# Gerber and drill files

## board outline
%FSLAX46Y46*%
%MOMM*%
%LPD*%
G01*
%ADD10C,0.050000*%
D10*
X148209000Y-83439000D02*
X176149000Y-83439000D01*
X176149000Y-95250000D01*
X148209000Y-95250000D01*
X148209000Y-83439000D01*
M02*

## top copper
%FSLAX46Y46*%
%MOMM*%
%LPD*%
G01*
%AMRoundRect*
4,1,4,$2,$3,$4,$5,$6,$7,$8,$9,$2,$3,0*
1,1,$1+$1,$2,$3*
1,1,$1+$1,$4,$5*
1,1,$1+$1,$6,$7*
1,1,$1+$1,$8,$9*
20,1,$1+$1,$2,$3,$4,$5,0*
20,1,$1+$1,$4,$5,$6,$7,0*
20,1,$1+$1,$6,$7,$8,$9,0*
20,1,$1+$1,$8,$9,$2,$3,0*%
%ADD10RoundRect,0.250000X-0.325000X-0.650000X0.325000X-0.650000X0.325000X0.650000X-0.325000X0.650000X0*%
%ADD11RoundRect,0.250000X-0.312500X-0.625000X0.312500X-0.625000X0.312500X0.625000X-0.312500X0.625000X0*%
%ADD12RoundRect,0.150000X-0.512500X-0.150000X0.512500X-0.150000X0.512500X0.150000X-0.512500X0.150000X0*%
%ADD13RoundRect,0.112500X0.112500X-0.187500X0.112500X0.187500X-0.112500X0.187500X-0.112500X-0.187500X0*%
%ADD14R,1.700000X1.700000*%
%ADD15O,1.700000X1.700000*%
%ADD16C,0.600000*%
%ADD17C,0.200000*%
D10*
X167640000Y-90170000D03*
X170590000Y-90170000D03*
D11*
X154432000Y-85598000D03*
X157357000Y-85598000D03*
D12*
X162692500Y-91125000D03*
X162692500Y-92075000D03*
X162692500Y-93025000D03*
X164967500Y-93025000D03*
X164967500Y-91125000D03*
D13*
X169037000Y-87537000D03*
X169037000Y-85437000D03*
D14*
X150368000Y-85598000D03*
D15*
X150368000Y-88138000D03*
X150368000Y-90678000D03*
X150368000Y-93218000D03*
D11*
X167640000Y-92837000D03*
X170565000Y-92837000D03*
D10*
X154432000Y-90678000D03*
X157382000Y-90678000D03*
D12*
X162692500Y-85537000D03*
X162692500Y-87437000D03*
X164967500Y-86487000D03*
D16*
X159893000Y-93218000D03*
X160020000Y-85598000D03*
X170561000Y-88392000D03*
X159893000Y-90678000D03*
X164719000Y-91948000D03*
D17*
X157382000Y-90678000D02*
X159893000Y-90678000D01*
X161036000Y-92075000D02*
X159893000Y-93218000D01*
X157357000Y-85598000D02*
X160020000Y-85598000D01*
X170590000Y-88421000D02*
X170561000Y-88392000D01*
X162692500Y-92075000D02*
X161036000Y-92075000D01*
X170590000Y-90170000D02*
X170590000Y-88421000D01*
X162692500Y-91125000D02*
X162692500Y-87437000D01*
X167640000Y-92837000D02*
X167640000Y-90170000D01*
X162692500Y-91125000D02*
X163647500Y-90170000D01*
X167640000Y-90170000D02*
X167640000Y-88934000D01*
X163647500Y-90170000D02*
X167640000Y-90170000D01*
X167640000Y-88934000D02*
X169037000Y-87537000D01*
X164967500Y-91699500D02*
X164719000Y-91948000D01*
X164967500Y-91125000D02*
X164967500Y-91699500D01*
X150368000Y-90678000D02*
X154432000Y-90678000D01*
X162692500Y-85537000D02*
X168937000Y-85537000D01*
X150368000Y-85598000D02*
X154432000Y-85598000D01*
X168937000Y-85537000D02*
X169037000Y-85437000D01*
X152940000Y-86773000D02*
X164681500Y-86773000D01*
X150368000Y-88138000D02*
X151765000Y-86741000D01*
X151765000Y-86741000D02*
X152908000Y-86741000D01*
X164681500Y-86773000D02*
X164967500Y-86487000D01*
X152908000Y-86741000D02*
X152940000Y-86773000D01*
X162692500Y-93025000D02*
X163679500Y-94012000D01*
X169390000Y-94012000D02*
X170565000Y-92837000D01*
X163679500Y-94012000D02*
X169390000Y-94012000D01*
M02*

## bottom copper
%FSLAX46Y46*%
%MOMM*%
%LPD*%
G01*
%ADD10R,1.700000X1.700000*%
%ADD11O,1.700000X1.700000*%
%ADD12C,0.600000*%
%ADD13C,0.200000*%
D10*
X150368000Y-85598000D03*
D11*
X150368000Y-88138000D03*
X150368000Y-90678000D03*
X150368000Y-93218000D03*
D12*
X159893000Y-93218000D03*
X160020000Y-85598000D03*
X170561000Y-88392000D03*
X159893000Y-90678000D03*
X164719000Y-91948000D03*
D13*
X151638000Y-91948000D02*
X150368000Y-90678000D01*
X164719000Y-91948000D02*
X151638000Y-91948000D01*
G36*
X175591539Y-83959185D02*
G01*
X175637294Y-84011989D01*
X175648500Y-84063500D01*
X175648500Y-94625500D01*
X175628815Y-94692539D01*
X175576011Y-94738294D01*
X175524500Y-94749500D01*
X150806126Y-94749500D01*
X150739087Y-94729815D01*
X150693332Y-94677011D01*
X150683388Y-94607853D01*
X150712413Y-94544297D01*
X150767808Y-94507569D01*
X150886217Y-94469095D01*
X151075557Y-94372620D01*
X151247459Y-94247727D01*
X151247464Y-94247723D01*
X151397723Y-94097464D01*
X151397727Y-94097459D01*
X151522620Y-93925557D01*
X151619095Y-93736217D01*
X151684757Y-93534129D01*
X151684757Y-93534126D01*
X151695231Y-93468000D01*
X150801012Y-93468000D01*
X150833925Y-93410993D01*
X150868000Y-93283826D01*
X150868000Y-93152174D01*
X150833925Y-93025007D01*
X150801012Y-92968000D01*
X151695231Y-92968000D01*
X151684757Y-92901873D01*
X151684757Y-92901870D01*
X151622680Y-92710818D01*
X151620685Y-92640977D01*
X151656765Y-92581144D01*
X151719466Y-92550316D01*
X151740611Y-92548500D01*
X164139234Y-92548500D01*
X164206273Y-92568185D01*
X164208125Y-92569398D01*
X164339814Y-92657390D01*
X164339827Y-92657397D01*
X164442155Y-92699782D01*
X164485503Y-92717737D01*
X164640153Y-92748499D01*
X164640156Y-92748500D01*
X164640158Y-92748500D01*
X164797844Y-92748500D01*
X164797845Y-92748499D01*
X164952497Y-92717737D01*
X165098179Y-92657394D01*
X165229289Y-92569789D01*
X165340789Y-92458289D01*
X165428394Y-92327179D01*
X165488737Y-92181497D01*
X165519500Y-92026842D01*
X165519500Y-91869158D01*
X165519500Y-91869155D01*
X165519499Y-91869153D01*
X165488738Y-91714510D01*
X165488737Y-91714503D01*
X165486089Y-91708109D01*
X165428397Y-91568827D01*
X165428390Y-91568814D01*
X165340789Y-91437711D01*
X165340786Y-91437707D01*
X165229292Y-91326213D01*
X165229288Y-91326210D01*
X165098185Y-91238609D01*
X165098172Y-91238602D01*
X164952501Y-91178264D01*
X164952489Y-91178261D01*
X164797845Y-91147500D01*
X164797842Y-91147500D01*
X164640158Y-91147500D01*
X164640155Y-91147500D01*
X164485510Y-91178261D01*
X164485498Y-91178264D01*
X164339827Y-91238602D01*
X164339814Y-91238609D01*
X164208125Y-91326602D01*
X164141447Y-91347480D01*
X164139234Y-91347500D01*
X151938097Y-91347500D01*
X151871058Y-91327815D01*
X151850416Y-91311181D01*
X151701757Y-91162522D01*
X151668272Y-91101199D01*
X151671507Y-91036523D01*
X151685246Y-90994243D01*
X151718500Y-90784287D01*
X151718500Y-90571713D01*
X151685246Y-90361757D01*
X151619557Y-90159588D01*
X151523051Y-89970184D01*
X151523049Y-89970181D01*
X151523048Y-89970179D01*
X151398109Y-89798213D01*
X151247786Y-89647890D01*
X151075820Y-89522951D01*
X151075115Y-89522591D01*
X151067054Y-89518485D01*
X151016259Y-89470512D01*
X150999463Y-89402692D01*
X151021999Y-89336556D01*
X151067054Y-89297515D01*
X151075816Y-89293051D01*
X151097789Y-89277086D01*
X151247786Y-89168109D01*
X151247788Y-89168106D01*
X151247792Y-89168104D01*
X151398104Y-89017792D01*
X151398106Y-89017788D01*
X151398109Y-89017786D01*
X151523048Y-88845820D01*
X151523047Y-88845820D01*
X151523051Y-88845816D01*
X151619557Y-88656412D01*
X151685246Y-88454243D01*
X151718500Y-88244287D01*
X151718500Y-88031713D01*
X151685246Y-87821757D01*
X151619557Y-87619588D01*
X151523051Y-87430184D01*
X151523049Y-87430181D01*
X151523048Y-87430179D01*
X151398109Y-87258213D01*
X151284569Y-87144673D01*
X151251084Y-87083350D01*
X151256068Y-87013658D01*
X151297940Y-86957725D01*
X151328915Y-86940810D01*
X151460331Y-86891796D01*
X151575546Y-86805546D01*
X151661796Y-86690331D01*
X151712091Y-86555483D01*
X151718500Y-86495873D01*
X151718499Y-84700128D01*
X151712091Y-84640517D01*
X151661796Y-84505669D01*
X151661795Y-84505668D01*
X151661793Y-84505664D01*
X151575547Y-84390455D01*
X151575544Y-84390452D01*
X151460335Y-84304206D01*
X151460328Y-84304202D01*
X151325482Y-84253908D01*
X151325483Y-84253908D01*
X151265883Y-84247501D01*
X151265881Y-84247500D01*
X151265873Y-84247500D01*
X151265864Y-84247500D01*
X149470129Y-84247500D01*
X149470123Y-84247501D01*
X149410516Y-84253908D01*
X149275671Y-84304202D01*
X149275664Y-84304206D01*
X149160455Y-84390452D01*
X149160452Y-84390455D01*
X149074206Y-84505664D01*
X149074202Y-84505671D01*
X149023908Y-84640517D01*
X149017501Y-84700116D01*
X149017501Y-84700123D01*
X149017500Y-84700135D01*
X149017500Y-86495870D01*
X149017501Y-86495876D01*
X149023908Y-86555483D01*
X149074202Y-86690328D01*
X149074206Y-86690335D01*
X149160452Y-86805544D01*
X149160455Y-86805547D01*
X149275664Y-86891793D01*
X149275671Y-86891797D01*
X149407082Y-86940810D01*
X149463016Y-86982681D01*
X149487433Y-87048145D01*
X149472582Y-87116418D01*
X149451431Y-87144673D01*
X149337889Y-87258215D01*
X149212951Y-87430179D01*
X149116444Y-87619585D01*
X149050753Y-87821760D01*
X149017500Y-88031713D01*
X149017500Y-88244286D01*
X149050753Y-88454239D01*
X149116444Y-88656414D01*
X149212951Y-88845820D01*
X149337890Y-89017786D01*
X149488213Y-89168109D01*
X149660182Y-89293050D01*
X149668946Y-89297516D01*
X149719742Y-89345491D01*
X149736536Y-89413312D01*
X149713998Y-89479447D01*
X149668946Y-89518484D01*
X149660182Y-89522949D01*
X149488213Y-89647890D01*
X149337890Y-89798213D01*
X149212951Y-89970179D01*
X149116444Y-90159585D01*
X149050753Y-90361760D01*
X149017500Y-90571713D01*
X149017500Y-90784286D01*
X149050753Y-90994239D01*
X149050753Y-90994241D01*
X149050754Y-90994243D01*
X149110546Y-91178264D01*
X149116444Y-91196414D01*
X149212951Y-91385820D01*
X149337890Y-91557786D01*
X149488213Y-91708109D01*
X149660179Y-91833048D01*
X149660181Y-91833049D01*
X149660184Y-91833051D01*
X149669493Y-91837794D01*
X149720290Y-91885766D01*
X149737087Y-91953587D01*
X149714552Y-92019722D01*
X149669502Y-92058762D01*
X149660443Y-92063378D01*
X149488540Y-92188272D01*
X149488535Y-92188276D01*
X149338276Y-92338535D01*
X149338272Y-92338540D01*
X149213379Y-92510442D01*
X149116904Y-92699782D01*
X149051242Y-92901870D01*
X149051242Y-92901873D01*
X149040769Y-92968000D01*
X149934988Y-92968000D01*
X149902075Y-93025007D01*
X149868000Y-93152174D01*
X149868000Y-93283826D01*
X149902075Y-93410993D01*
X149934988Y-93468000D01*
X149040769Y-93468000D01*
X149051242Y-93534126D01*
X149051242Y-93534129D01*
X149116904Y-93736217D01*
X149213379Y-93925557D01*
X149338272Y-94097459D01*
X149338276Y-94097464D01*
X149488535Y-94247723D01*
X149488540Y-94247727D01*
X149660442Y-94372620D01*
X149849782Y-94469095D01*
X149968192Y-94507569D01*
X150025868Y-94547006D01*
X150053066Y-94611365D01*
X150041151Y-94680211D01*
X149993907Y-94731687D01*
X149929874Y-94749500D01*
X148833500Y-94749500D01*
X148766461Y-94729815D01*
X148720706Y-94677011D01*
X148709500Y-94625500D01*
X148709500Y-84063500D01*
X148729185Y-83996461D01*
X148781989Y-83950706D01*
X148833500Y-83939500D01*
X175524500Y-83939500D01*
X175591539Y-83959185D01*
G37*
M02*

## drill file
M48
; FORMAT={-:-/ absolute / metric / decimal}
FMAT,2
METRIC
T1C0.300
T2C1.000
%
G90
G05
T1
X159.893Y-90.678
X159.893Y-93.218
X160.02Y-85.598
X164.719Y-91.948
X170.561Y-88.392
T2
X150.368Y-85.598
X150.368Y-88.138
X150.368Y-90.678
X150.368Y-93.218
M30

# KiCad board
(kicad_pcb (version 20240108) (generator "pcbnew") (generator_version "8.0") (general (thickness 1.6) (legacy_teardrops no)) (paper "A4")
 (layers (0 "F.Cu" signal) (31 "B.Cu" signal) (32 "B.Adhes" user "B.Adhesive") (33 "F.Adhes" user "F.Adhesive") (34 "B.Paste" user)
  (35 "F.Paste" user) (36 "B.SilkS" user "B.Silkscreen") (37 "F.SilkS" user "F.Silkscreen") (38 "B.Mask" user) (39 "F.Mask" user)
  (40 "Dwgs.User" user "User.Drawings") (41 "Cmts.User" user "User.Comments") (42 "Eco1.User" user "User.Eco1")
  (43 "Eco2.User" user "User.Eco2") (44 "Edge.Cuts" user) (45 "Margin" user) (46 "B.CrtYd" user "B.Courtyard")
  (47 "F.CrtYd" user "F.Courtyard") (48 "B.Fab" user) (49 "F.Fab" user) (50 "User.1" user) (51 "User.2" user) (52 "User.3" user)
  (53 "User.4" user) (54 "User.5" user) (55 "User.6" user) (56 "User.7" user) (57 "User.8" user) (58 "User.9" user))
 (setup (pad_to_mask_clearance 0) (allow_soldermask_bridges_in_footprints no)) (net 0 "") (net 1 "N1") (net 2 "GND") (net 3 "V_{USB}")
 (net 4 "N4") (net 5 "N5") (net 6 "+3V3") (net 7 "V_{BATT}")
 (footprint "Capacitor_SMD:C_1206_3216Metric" (layer "F.Cu") (at 169.115 90.17)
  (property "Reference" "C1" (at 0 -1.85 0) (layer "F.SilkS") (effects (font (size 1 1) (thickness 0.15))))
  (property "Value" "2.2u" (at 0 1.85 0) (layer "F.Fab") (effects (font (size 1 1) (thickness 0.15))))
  (pad "1" smd roundrect (at -1.475 0) (size 1.15 1.8) (layers "F.Cu" "F.Paste" "F.Mask") (roundrect_rratio 0.217391) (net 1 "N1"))
  (pad "2" smd roundrect (at 1.475 0) (size 1.15 1.8) (layers "F.Cu" "F.Paste" "F.Mask") (roundrect_rratio 0.217391) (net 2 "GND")))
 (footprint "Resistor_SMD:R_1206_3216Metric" (layer "F.Cu") (at 155.8945 85.598)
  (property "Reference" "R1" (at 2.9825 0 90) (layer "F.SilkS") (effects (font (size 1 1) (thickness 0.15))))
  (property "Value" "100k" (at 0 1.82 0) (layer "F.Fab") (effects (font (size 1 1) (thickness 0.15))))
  (pad "1" smd roundrect (at -1.4625 0) (size 1.125 1.75) (layers "F.Cu" "F.Paste" "F.Mask") (roundrect_rratio 0.222222) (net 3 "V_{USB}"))
  (pad "2" smd roundrect (at 1.4625 0) (size 1.125 1.75) (layers "F.Cu" "F.Paste" "F.Mask") (roundrect_rratio 0.222222) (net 2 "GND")))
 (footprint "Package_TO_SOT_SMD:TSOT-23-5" (layer "F.Cu") (at 163.83 92.075)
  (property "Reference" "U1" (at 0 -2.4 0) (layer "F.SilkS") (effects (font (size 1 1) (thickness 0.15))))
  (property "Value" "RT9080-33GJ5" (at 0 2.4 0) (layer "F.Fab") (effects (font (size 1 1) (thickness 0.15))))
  (pad "1" smd roundrect (at -1.1375 -0.95) (size 1.325 0.6) (layers "F.Cu" "F.Paste" "F.Mask") (roundrect_rratio 0.25) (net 1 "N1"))
  (pad "2" smd roundrect (at -1.1375 0) (size 1.325 0.6) (layers "F.Cu" "F.Paste" "F.Mask") (roundrect_rratio 0.25) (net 2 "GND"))
  (pad "3" smd roundrect (at -1.1375 0.95) (size 1.325 0.6) (layers "F.Cu" "F.Paste" "F.Mask") (roundrect_rratio 0.25) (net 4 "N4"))
  (pad "4" smd roundrect (at 1.1375 0.95) (size 1.325 0.6) (layers "F.Cu" "F.Paste" "F.Mask") (roundrect_rratio 0.25) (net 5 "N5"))
  (pad "5" smd roundrect (at 1.1375 -0.95) (size 1.325 0.6) (layers "F.Cu" "F.Paste" "F.Mask") (roundrect_rratio 0.25) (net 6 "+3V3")))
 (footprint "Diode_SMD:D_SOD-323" (layer "F.Cu") (at 169.037 86.487 90)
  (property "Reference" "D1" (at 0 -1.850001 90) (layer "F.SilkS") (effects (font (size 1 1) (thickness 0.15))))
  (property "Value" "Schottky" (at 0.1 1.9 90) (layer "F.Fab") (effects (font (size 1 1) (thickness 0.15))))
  (pad "1" smd roundrect (at -1.05 0 90) (size 0.6 0.45) (layers "F.Cu" "F.Paste" "F.Mask") (roundrect_rratio 0.25) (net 1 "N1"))
  (pad "2" smd roundrect (at 1.05 0 90) (size 0.6 0.45) (layers "F.Cu" "F.Paste" "F.Mask") (roundrect_rratio 0.25) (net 3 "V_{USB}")))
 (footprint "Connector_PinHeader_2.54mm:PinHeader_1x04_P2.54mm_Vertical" (layer "F.Cu") (at 150.368 85.598)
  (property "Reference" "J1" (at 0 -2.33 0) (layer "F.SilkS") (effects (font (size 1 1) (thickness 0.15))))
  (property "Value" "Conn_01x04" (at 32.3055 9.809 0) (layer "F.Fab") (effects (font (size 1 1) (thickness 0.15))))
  (pad "1" thru_hole rect (at 0 0) (size 1.7 1.7) (drill 1) (layers "*.Cu" "*.Mask") (remove_unused_layers no) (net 3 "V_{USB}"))
  (pad "2" thru_hole oval (at 0 2.54) (size 1.7 1.7) (drill 1) (layers "*.Cu" "*.Mask") (remove_unused_layers no) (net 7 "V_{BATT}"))
  (pad "3" thru_hole oval (at 0 5.08) (size 1.7 1.7) (drill 1) (layers "*.Cu" "*.Mask") (remove_unused_layers no) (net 6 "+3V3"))
  (pad "4" thru_hole oval (at 0 7.62) (size 1.7 1.7) (drill 1) (layers "*.Cu" "*.Mask") (remove_unused_layers no) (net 2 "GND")))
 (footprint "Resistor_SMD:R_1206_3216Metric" (layer "F.Cu") (at 169.1025 92.837)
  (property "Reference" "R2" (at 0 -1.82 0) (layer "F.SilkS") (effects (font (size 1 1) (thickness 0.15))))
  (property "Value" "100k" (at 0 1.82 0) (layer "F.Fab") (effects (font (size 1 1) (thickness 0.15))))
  (pad "1" smd roundrect (at -1.4625 0) (size 1.125 1.75) (layers "F.Cu" "F.Paste" "F.Mask") (roundrect_rratio 0.222222) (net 1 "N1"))
  (pad "2" smd roundrect (at 1.4625 0) (size 1.125 1.75) (layers "F.Cu" "F.Paste" "F.Mask") (roundrect_rratio 0.222222) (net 4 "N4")))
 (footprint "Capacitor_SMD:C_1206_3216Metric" (layer "F.Cu") (at 155.907 90.678)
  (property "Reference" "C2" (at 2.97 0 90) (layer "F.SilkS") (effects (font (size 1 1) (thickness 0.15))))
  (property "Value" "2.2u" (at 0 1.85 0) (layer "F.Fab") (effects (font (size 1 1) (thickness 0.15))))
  (pad "1" smd roundrect (at -1.475 0) (size 1.15 1.8) (layers "F.Cu" "F.Paste" "F.Mask") (roundrect_rratio 0.217391) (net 6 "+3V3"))
  (pad "2" smd roundrect (at 1.475 0) (size 1.15 1.8) (layers "F.Cu" "F.Paste" "F.Mask") (roundrect_rratio 0.217391) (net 2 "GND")))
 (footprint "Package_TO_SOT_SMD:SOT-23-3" (layer "F.Cu") (at 163.83 86.487)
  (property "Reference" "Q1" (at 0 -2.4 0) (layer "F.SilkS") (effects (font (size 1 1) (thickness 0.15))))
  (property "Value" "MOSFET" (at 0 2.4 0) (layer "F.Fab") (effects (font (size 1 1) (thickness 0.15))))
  (pad "1" smd roundrect (at -1.1375 -0.95) (size 1.325 0.6) (layers "F.Cu" "F.Paste" "F.Mask") (roundrect_rratio 0.25) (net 3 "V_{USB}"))
  (pad "2" smd roundrect (at -1.1375 0.95) (size 1.325 0.6) (layers "F.Cu" "F.Paste" "F.Mask") (roundrect_rratio 0.25) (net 1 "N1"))
  (pad "3" smd roundrect (at 1.1375 0) (size 1.325 0.6) (layers "F.Cu" "F.Paste" "F.Mask") (roundrect_rratio 0.25) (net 7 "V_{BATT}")))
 (gr_rect (start 148.209 83.439) (end 176.149 95.25) (stroke (width 0.05) (type default)) (fill none) (layer "Edge.Cuts"))
 (segment (start 157.382 90.678) (end 159.893 90.678) (width 0.2) (layer "F.Cu") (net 2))
 (segment (start 161.036 92.075) (end 159.893 93.218) (width 0.2) (layer "F.Cu") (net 2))
 (segment (start 157.357 85.598) (end 160.02 85.598) (width 0.2) (layer "F.Cu") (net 2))
 (segment (start 170.59 88.421) (end 170.561 88.392) (width 0.2) (layer "F.Cu") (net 2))
 (segment (start 162.6925 92.075) (end 161.036 92.075) (width 0.2) (layer "F.Cu") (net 2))
 (segment (start 170.59 90.17) (end 170.59 88.421) (width 0.2) (layer "F.Cu") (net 2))
 (via (at 159.893 93.218) (size 0.6) (drill 0.3) (layers "F.Cu" "B.Cu") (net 2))
 (via (at 160.02 85.598) (size 0.6) (drill 0.3) (layers "F.Cu" "B.Cu") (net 2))
 (via (at 170.561 88.392) (size 0.6) (drill 0.3) (layers "F.Cu" "B.Cu") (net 2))
 (via (at 159.893 90.678) (size 0.6) (drill 0.3) (layers "F.Cu" "B.Cu") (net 2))
 (segment (start 162.6925 91.125) (end 162.6925 87.437) (width 0.2) (layer "F.Cu") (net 1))
 (segment (start 167.64 92.837) (end 167.64 90.17) (width 0.2) (layer "F.Cu") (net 1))
 (segment (start 162.6925 91.125) (end 163.6475 90.17) (width 0.2) (layer "F.Cu") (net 1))
 (segment (start 167.64 90.17) (end 167.64 88.934) (width 0.2) (layer "F.Cu") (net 1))
 (segment (start 163.6475 90.17) (end 167.64 90.17) (width 0.2) (layer "F.Cu") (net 1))
 (segment (start 167.64 88.934) (end 169.037 87.537) (width 0.2) (layer "F.Cu") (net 1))
 (segment (start 164.9675 91.6995) (end 164.719 91.948) (width 0.2) (layer "F.Cu") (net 6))
 (segment (start 164.9675 91.125) (end 164.9675 91.6995) (width 0.2) (layer "F.Cu") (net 6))
 (segment (start 150.368 90.678) (end 154.432 90.678) (width 0.2) (layer "F.Cu") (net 6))
 (via (at 164.719 91.948) (size 0.6) (drill 0.3) (layers "F.Cu" "B.Cu") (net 6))
 (segment (start 151.638 91.948) (end 150.368 90.678) (width 0.2) (layer "B.Cu") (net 6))
 (segment (start 164.719 91.948) (end 151.638 91.948) (width 0.2) (layer "B.Cu") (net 6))
 (segment (start 162.6925 85.537) (end 168.937 85.537) (width 0.2) (layer "F.Cu") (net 3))
 (segment (start 150.368 85.598) (end 154.432 85.598) (width 0.2) (layer "F.Cu") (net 3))
 (segment (start 168.937 85.537) (end 169.037 85.437) (width 0.2) (layer "F.Cu") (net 3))
 (segment (start 152.94 86.773) (end 164.6815 86.773) (width 0.2) (layer "F.Cu") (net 7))
 (segment (start 150.368 88.138) (end 151.765 86.741) (width 0.2) (layer "F.Cu") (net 7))
 (segment (start 151.765 86.741) (end 152.908 86.741) (width 0.2) (layer "F.Cu") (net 7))
 (segment (start 164.6815 86.773) (end 164.9675 86.487) (width 0.2) (layer "F.Cu") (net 7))
 (segment (start 152.908 86.741) (end 152.94 86.773) (width 0.2) (layer "F.Cu") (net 7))
 (segment (start 162.6925 93.025) (end 163.6795 94.012) (width 0.2) (layer "F.Cu") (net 4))
 (segment (start 169.39 94.012) (end 170.565 92.837) (width 0.2) (layer "F.Cu") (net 4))
 (segment (start 163.6795 94.012) (end 169.39 94.012) (width 0.2) (layer "F.Cu") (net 4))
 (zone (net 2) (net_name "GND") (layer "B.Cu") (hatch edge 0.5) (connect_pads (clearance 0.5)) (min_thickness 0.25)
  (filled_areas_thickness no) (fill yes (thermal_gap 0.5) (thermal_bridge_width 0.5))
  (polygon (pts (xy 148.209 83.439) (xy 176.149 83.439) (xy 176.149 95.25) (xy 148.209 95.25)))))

